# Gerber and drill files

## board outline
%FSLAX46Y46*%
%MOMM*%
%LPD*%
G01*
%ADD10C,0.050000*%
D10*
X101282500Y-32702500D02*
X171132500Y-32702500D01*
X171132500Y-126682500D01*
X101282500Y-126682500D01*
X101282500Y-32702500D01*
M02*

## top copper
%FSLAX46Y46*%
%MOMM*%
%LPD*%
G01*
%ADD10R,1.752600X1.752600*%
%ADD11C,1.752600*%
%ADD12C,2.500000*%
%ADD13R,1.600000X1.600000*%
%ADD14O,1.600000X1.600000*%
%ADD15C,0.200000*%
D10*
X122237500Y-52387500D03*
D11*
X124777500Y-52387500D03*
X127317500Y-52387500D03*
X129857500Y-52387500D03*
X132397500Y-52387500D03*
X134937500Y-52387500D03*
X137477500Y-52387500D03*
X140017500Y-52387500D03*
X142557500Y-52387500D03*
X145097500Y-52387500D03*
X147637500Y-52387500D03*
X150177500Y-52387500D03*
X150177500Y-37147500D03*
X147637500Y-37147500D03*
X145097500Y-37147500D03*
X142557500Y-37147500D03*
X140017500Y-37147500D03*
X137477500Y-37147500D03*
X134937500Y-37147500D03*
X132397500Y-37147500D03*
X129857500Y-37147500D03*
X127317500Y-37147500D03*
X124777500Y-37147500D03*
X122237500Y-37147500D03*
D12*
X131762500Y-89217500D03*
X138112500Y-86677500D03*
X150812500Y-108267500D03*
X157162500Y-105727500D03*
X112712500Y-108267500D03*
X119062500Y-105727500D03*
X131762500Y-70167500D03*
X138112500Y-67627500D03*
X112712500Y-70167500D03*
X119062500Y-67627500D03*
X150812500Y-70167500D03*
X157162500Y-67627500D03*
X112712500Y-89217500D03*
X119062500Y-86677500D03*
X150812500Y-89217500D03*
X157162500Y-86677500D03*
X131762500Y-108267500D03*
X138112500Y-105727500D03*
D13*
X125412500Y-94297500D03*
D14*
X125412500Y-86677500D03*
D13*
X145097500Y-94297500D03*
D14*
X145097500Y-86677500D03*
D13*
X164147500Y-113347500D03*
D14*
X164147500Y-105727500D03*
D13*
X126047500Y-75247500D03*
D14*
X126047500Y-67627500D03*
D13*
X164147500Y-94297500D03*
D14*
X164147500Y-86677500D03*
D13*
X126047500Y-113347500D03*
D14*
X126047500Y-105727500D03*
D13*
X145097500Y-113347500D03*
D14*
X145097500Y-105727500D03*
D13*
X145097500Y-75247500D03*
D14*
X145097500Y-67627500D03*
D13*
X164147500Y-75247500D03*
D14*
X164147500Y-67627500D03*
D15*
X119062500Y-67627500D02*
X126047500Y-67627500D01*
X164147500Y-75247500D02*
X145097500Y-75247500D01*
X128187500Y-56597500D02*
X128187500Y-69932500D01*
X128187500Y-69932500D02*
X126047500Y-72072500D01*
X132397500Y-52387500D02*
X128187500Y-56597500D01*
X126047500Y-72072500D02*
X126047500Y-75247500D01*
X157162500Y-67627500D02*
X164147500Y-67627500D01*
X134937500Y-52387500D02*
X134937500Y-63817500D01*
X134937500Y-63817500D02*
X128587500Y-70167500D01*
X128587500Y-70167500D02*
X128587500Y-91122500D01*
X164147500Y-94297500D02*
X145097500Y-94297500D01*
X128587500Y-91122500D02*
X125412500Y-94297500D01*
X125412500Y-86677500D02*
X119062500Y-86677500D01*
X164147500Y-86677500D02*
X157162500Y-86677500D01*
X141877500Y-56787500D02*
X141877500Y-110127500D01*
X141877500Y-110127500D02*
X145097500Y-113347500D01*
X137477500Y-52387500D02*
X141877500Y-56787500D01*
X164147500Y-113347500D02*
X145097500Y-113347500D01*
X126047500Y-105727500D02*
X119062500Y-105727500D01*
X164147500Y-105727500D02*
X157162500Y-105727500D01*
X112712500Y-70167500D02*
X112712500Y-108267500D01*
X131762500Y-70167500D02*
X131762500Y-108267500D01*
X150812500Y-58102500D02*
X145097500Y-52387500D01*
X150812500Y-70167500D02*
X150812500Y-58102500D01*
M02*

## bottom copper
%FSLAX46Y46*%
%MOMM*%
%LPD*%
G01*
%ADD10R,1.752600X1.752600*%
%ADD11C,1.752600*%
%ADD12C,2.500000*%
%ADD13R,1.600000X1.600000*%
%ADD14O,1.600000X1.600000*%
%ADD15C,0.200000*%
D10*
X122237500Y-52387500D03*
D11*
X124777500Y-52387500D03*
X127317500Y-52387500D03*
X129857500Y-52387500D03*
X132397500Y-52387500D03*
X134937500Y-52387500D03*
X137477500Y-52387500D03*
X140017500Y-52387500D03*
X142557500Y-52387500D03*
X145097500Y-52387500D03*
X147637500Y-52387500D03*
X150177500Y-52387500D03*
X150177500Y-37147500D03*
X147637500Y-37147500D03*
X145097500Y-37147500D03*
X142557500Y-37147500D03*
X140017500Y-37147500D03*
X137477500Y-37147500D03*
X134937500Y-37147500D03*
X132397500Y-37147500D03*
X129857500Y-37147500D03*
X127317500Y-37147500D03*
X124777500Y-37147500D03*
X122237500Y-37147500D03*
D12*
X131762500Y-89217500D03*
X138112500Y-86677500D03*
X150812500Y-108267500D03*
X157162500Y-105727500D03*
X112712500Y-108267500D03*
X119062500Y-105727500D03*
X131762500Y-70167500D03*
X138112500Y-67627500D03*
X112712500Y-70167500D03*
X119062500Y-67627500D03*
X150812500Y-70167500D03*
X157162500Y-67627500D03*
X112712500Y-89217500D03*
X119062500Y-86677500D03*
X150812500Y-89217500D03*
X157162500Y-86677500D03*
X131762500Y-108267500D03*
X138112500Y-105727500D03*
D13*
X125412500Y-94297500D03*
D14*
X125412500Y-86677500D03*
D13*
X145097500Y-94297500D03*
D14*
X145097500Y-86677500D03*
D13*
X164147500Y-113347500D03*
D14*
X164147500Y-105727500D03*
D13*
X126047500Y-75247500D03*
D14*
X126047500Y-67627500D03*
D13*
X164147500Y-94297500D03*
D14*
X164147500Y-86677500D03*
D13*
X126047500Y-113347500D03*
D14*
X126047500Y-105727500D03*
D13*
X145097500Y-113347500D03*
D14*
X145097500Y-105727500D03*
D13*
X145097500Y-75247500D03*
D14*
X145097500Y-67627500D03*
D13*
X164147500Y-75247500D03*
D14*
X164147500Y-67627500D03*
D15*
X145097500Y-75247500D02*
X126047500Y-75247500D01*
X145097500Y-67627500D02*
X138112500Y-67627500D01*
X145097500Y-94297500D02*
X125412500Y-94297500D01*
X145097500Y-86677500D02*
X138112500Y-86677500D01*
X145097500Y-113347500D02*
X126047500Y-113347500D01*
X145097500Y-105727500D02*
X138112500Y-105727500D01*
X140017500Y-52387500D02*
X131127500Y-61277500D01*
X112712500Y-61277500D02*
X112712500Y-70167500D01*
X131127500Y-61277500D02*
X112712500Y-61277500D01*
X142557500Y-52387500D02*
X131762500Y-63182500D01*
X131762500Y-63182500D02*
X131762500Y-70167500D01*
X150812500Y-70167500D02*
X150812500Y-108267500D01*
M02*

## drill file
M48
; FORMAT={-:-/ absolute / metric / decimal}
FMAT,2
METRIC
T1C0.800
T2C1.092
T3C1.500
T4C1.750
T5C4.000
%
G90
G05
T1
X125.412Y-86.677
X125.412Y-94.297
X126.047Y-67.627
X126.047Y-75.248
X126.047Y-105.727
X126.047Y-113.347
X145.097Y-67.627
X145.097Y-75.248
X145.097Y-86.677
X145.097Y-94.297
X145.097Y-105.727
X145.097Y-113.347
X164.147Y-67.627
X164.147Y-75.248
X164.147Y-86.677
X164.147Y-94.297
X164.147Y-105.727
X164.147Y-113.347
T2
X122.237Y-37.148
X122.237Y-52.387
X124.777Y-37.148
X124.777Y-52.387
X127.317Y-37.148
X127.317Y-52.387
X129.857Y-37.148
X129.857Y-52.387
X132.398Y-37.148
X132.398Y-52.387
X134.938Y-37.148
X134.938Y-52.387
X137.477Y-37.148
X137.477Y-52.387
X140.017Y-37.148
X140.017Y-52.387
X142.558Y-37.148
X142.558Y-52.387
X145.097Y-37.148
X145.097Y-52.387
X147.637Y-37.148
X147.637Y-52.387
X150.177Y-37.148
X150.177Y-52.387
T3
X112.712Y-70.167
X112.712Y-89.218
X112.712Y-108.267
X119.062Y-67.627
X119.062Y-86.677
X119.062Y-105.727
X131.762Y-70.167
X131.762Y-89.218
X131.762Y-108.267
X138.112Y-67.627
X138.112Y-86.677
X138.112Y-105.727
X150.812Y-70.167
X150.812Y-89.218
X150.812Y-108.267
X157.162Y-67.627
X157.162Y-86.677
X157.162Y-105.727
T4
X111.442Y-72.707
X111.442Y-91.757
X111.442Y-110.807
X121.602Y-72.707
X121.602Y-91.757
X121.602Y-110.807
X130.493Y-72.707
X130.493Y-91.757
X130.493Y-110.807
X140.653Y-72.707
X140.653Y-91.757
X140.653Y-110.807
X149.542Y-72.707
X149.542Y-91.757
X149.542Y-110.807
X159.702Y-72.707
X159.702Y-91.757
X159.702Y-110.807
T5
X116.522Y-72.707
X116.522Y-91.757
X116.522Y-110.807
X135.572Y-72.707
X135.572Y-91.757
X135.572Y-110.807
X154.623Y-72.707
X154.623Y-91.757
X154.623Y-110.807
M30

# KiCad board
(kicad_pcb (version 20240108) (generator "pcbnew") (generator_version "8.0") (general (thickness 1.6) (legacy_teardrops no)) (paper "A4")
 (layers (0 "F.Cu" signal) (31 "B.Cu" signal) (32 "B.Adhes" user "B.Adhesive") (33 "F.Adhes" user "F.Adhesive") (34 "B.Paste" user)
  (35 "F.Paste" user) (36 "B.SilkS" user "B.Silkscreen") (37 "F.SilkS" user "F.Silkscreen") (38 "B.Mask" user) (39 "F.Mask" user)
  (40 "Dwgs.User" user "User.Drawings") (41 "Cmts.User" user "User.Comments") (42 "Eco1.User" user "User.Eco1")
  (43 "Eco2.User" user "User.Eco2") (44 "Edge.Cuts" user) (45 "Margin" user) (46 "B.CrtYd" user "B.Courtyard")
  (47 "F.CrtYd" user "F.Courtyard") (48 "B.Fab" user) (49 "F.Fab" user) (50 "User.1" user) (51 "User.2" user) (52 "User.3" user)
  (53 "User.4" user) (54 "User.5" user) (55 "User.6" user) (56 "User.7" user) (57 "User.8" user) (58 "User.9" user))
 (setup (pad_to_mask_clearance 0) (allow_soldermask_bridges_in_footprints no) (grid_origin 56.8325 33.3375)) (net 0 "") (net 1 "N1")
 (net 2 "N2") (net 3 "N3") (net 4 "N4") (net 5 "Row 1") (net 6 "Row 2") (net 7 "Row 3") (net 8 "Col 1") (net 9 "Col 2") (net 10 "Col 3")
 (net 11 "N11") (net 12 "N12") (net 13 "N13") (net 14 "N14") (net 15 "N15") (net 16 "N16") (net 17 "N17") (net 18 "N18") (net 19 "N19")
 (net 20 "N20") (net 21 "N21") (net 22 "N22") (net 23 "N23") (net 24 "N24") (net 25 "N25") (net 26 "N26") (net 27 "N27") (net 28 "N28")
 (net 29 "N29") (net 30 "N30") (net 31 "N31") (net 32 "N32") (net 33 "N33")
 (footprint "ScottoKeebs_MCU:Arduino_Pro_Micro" (layer "F.Cu") (at 136.2075 44.7675 90)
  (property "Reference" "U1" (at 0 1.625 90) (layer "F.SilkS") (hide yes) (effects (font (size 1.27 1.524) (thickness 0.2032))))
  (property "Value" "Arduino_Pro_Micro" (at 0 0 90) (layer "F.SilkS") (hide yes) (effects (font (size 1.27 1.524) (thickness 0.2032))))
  (pad "1" thru_hole rect (at -7.62 -13.97) (size 1.7526 1.7526) (drill 1.0922) (layers "*.Cu" "*.SilkS" "*.Mask") (remove_unused_layers no)
   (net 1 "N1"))
  (pad "2" thru_hole circle (at -7.62 -11.43) (size 1.7526 1.7526) (drill 1.0922) (layers "*.Cu" "*.SilkS" "*.Mask")
   (remove_unused_layers no) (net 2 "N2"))
  (pad "3" thru_hole circle (at -7.62 -8.89) (size 1.7526 1.7526) (drill 1.0922) (layers "*.Cu" "*.SilkS" "*.Mask")
   (remove_unused_layers no) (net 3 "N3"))
  (pad "4" thru_hole circle (at -7.62 -6.35) (size 1.7526 1.7526) (drill 1.0922) (layers "*.Cu" "*.SilkS" "*.Mask")
   (remove_unused_layers no) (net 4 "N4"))
  (pad "5" thru_hole circle (at -7.62 -3.81) (size 1.7526 1.7526) (drill 1.0922) (layers "*.Cu" "*.SilkS" "*.Mask")
   (remove_unused_layers no) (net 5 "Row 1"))
  (pad "6" thru_hole circle (at -7.62 -1.27) (size 1.7526 1.7526) (drill 1.0922) (layers "*.Cu" "*.SilkS" "*.Mask")
   (remove_unused_layers no) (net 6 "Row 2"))
  (pad "7" thru_hole circle (at -7.62 1.27) (size 1.7526 1.7526) (drill 1.0922) (layers "*.Cu" "*.SilkS" "*.Mask") (remove_unused_layers no)
   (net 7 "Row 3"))
  (pad "8" thru_hole circle (at -7.62 3.81) (size 1.7526 1.7526) (drill 1.0922) (layers "*.Cu" "*.SilkS" "*.Mask") (remove_unused_layers no)
   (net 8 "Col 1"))
  (pad "9" thru_hole circle (at -7.62 6.35) (size 1.7526 1.7526) (drill 1.0922) (layers "*.Cu" "*.SilkS" "*.Mask") (remove_unused_layers no)
   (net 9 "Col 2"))
  (pad "10" thru_hole circle (at -7.62 8.89) (size 1.7526 1.7526) (drill 1.0922) (layers "*.Cu" "*.SilkS" "*.Mask")
   (remove_unused_layers no) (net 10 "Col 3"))
  (pad "11" thru_hole circle (at -7.62 11.43) (size 1.7526 1.7526) (drill 1.0922) (layers "*.Cu" "*.SilkS" "*.Mask")
   (remove_unused_layers no) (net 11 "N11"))
  (pad "12" thru_hole circle (at -7.62 13.97) (size 1.7526 1.7526) (drill 1.0922) (layers "*.Cu" "*.SilkS" "*.Mask")
   (remove_unused_layers no) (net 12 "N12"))
  (pad "13" thru_hole circle (at 7.62 13.97) (size 1.7526 1.7526) (drill 1.0922) (layers "*.Cu" "*.SilkS" "*.Mask")
   (remove_unused_layers no) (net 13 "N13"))
  (pad "14" thru_hole circle (at 7.62 11.43) (size 1.7526 1.7526) (drill 1.0922) (layers "*.Cu" "*.SilkS" "*.Mask")
   (remove_unused_layers no) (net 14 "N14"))
  (pad "15" thru_hole circle (at 7.62 8.89) (size 1.7526 1.7526) (drill 1.0922) (layers "*.Cu" "*.SilkS" "*.Mask") (remove_unused_layers no)
   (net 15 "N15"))
  (pad "16" thru_hole circle (at 7.62 6.35) (size 1.7526 1.7526) (drill 1.0922) (layers "*.Cu" "*.SilkS" "*.Mask") (remove_unused_layers no)
   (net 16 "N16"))
  (pad "17" thru_hole circle (at 7.62 3.81) (size 1.7526 1.7526) (drill 1.0922) (layers "*.Cu" "*.SilkS" "*.Mask") (remove_unused_layers no)
   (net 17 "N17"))
  (pad "18" thru_hole circle (at 7.62 1.27) (size 1.7526 1.7526) (drill 1.0922) (layers "*.Cu" "*.SilkS" "*.Mask") (remove_unused_layers no)
   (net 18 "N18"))
  (pad "19" thru_hole circle (at 7.62 -1.27) (size 1.7526 1.7526) (drill 1.0922) (layers "*.Cu" "*.SilkS" "*.Mask")
   (remove_unused_layers no) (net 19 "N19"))
  (pad "20" thru_hole circle (at 7.62 -3.81) (size 1.7526 1.7526) (drill 1.0922) (layers "*.Cu" "*.SilkS" "*.Mask")
   (remove_unused_layers no) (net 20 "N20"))
  (pad "21" thru_hole circle (at 7.62 -6.35) (size 1.7526 1.7526) (drill 1.0922) (layers "*.Cu" "*.SilkS" "*.Mask")
   (remove_unused_layers no) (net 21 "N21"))
  (pad "22" thru_hole circle (at 7.62 -8.89) (size 1.7526 1.7526) (drill 1.0922) (layers "*.Cu" "*.SilkS" "*.Mask")
   (remove_unused_layers no) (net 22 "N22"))
  (pad "23" thru_hole circle (at 7.62 -11.43) (size 1.7526 1.7526) (drill 1.0922) (layers "*.Cu" "*.SilkS" "*.Mask")
   (remove_unused_layers no) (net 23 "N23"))
  (pad "24" thru_hole circle (at 7.62 -13.97) (size 1.7526 1.7526) (drill 1.0922) (layers "*.Cu" "*.SilkS" "*.Mask")
   (remove_unused_layers no) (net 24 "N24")))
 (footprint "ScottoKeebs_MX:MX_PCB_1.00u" (layer "F.Cu") (at 135.5725 91.7575)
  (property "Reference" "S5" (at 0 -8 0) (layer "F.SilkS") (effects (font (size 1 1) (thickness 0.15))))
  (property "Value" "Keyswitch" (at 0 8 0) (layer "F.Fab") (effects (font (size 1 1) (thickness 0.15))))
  (pad "" np_thru_hole circle (at -5.08 0) (size 1.75 1.75) (drill 1.75) (layers "*.Cu" "*.Mask"))
  (pad "" np_thru_hole circle (at 0 0) (size 4 4) (drill 4) (layers "*.Cu" "*.Mask"))
  (pad "" np_thru_hole circle (at 5.08 0) (size 1.75 1.75) (drill 1.75) (layers "*.Cu" "*.Mask"))
  (pad "1" thru_hole circle (at -3.81 -2.54) (size 2.5 2.5) (drill 1.5) (layers "*.Cu" "*.Mask") (remove_unused_layers no) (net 9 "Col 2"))
  (pad "2" thru_hole circle (at 2.54 -5.08) (size 2.5 2.5) (drill 1.5) (layers "*.Cu" "*.Mask") (remove_unused_layers no) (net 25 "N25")))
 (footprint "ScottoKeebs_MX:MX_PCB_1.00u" (layer "F.Cu") (at 154.6225 110.8075)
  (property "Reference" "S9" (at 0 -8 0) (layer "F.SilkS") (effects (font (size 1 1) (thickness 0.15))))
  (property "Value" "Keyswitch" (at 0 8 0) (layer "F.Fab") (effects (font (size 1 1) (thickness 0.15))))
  (pad "" np_thru_hole circle (at -5.08 0) (size 1.75 1.75) (drill 1.75) (layers "*.Cu" "*.Mask"))
  (pad "" np_thru_hole circle (at 0 0) (size 4 4) (drill 4) (layers "*.Cu" "*.Mask"))
  (pad "" np_thru_hole circle (at 5.08 0) (size 1.75 1.75) (drill 1.75) (layers "*.Cu" "*.Mask"))
  (pad "1" thru_hole circle (at -3.81 -2.54) (size 2.5 2.5) (drill 1.5) (layers "*.Cu" "*.Mask") (remove_unused_layers no) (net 10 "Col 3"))
  (pad "2" thru_hole circle (at 2.54 -5.08) (size 2.5 2.5) (drill 1.5) (layers "*.Cu" "*.Mask") (remove_unused_layers no) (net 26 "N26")))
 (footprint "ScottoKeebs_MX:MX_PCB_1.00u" (layer "F.Cu") (at 116.5225 110.8075)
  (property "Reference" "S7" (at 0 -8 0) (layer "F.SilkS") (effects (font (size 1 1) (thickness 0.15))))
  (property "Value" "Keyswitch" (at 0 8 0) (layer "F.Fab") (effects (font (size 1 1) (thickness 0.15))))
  (pad "" np_thru_hole circle (at -5.08 0) (size 1.75 1.75) (drill 1.75) (layers "*.Cu" "*.Mask"))
  (pad "" np_thru_hole circle (at 0 0) (size 4 4) (drill 4) (layers "*.Cu" "*.Mask"))
  (pad "" np_thru_hole circle (at 5.08 0) (size 1.75 1.75) (drill 1.75) (layers "*.Cu" "*.Mask"))
  (pad "1" thru_hole circle (at -3.81 -2.54) (size 2.5 2.5) (drill 1.5) (layers "*.Cu" "*.Mask") (remove_unused_layers no) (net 8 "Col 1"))
  (pad "2" thru_hole circle (at 2.54 -5.08) (size 2.5 2.5) (drill 1.5) (layers "*.Cu" "*.Mask") (remove_unused_layers no) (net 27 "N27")))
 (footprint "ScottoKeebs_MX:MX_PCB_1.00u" (layer "F.Cu") (at 135.5725 72.7075)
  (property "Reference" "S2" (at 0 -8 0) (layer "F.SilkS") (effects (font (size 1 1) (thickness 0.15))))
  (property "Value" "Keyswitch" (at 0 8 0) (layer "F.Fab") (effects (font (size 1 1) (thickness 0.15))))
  (pad "" np_thru_hole circle (at -5.08 0) (size 1.75 1.75) (drill 1.75) (layers "*.Cu" "*.Mask"))
  (pad "" np_thru_hole circle (at 0 0) (size 4 4) (drill 4) (layers "*.Cu" "*.Mask"))
  (pad "" np_thru_hole circle (at 5.08 0) (size 1.75 1.75) (drill 1.75) (layers "*.Cu" "*.Mask"))
  (pad "1" thru_hole circle (at -3.81 -2.54) (size 2.5 2.5) (drill 1.5) (layers "*.Cu" "*.Mask") (remove_unused_layers no) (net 9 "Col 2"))
  (pad "2" thru_hole circle (at 2.54 -5.08) (size 2.5 2.5) (drill 1.5) (layers "*.Cu" "*.Mask") (remove_unused_layers no) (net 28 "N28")))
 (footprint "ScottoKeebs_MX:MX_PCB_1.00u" (layer "F.Cu") (at 116.5225 72.7075)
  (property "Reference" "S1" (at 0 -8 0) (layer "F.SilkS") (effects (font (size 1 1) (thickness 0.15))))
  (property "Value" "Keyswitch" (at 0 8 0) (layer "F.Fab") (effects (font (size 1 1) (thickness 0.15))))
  (pad "" np_thru_hole circle (at -5.08 0) (size 1.75 1.75) (drill 1.75) (layers "*.Cu" "*.Mask"))
  (pad "" np_thru_hole circle (at 0 0) (size 4 4) (drill 4) (layers "*.Cu" "*.Mask"))
  (pad "" np_thru_hole circle (at 5.08 0) (size 1.75 1.75) (drill 1.75) (layers "*.Cu" "*.Mask"))
  (pad "1" thru_hole circle (at -3.81 -2.54) (size 2.5 2.5) (drill 1.5) (layers "*.Cu" "*.Mask") (remove_unused_layers no) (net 8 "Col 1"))
  (pad "2" thru_hole circle (at 2.54 -5.08) (size 2.5 2.5) (drill 1.5) (layers "*.Cu" "*.Mask") (remove_unused_layers no) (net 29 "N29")))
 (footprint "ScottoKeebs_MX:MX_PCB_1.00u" (layer "F.Cu") (at 154.6225 72.7075)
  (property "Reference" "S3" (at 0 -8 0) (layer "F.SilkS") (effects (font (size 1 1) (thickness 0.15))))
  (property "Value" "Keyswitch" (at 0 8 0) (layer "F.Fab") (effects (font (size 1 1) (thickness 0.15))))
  (pad "" np_thru_hole circle (at -5.08 0) (size 1.75 1.75) (drill 1.75) (layers "*.Cu" "*.Mask"))
  (pad "" np_thru_hole circle (at 0 0) (size 4 4) (drill 4) (layers "*.Cu" "*.Mask"))
  (pad "" np_thru_hole circle (at 5.08 0) (size 1.75 1.75) (drill 1.75) (layers "*.Cu" "*.Mask"))
  (pad "1" thru_hole circle (at -3.81 -2.54) (size 2.5 2.5) (drill 1.5) (layers "*.Cu" "*.Mask") (remove_unused_layers no) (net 10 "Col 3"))
  (pad "2" thru_hole circle (at 2.54 -5.08) (size 2.5 2.5) (drill 1.5) (layers "*.Cu" "*.Mask") (remove_unused_layers no) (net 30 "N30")))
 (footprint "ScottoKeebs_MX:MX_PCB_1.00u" (layer "F.Cu") (at 116.5225 91.7575)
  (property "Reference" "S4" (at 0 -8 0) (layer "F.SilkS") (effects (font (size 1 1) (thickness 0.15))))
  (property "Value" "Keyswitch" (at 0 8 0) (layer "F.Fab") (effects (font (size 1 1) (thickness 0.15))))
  (pad "" np_thru_hole circle (at -5.08 0) (size 1.75 1.75) (drill 1.75) (layers "*.Cu" "*.Mask"))
  (pad "" np_thru_hole circle (at 0 0) (size 4 4) (drill 4) (layers "*.Cu" "*.Mask"))
  (pad "" np_thru_hole circle (at 5.08 0) (size 1.75 1.75) (drill 1.75) (layers "*.Cu" "*.Mask"))
  (pad "1" thru_hole circle (at -3.81 -2.54) (size 2.5 2.5) (drill 1.5) (layers "*.Cu" "*.Mask") (remove_unused_layers no) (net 8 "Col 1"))
  (pad "2" thru_hole circle (at 2.54 -5.08) (size 2.5 2.5) (drill 1.5) (layers "*.Cu" "*.Mask") (remove_unused_layers no) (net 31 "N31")))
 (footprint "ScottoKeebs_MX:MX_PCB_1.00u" (layer "F.Cu") (at 154.6225 91.7575)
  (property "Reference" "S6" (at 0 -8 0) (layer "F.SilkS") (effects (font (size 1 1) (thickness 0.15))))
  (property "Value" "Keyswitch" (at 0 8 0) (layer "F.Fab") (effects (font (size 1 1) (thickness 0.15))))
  (pad "" np_thru_hole circle (at -5.08 0) (size 1.75 1.75) (drill 1.75) (layers "*.Cu" "*.Mask"))
  (pad "" np_thru_hole circle (at 0 0) (size 4 4) (drill 4) (layers "*.Cu" "*.Mask"))
  (pad "" np_thru_hole circle (at 5.08 0) (size 1.75 1.75) (drill 1.75) (layers "*.Cu" "*.Mask"))
  (pad "1" thru_hole circle (at -3.81 -2.54) (size 2.5 2.5) (drill 1.5) (layers "*.Cu" "*.Mask") (remove_unused_layers no) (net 10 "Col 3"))
  (pad "2" thru_hole circle (at 2.54 -5.08) (size 2.5 2.5) (drill 1.5) (layers "*.Cu" "*.Mask") (remove_unused_layers no) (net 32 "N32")))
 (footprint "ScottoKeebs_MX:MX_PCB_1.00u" (layer "F.Cu") (at 135.5725 110.8075)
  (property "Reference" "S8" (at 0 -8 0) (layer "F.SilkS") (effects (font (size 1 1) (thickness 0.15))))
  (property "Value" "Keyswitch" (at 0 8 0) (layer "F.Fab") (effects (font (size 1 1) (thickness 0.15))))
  (pad "" np_thru_hole circle (at -5.08 0) (size 1.75 1.75) (drill 1.75) (layers "*.Cu" "*.Mask"))
  (pad "" np_thru_hole circle (at 0 0) (size 4 4) (drill 4) (layers "*.Cu" "*.Mask"))
  (pad "" np_thru_hole circle (at 5.08 0) (size 1.75 1.75) (drill 1.75) (layers "*.Cu" "*.Mask"))
  (pad "1" thru_hole circle (at -3.81 -2.54) (size 2.5 2.5) (drill 1.5) (layers "*.Cu" "*.Mask") (remove_unused_layers no) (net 9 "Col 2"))
  (pad "2" thru_hole circle (at 2.54 -5.08) (size 2.5 2.5) (drill 1.5) (layers "*.Cu" "*.Mask") (remove_unused_layers no) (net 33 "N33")))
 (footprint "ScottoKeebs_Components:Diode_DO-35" (layer "B.Cu") (at 125.4125 94.2975 90)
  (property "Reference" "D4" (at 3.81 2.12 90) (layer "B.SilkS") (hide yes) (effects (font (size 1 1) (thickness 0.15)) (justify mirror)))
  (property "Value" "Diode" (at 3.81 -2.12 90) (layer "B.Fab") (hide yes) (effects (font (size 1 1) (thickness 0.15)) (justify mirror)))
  (pad "1" thru_hole rect (at 0 0 90) (size 1.6 1.6) (drill 0.8) (layers "*.Cu" "*.Mask") (remove_unused_layers no) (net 6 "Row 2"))
  (pad "2" thru_hole oval (at 7.62 0 90) (size 1.6 1.6) (drill 0.8) (layers "*.Cu" "*.Mask") (remove_unused_layers no) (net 31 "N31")))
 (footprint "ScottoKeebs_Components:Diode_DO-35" (layer "B.Cu") (at 145.0975 94.2975 90)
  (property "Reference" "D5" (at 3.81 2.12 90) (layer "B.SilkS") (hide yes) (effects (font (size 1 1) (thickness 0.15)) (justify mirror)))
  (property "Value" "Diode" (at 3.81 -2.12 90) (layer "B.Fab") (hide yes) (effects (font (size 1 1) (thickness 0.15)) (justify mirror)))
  (pad "1" thru_hole rect (at 0 0 90) (size 1.6 1.6) (drill 0.8) (layers "*.Cu" "*.Mask") (remove_unused_layers no) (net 6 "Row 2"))
  (pad "2" thru_hole oval (at 7.62 0 90) (size 1.6 1.6) (drill 0.8) (layers "*.Cu" "*.Mask") (remove_unused_layers no) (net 25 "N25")))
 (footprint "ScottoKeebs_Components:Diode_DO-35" (layer "B.Cu") (at 164.1475 113.3475 90)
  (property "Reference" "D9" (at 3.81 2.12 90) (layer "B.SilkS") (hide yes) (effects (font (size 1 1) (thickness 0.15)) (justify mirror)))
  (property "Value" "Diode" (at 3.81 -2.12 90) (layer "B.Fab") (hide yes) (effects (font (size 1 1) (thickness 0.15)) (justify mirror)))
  (pad "1" thru_hole rect (at 0 0 90) (size 1.6 1.6) (drill 0.8) (layers "*.Cu" "*.Mask") (remove_unused_layers no) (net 7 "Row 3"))
  (pad "2" thru_hole oval (at 7.62 0 90) (size 1.6 1.6) (drill 0.8) (layers "*.Cu" "*.Mask") (remove_unused_layers no) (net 26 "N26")))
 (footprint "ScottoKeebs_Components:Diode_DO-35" (layer "B.Cu") (at 126.0475 75.2475 90)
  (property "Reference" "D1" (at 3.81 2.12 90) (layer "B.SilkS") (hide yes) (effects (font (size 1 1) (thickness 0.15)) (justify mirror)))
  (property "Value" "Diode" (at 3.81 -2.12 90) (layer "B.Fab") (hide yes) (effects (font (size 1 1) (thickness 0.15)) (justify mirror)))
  (pad "1" thru_hole rect (at 0 0 90) (size 1.6 1.6) (drill 0.8) (layers "*.Cu" "*.Mask") (remove_unused_layers no) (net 5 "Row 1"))
  (pad "2" thru_hole oval (at 7.62 0 90) (size 1.6 1.6) (drill 0.8) (layers "*.Cu" "*.Mask") (remove_unused_layers no) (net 29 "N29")))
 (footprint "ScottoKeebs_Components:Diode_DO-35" (layer "B.Cu") (at 164.1475 94.2975 90)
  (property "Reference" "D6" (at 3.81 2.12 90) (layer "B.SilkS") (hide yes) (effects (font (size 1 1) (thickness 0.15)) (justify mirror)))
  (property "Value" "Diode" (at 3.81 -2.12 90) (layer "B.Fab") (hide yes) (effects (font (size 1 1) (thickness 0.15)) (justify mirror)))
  (pad "1" thru_hole rect (at 0 0 90) (size 1.6 1.6) (drill 0.8) (layers "*.Cu" "*.Mask") (remove_unused_layers no) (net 6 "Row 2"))
  (pad "2" thru_hole oval (at 7.62 0 90) (size 1.6 1.6) (drill 0.8) (layers "*.Cu" "*.Mask") (remove_unused_layers no) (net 32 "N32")))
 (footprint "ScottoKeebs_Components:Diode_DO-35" (layer "B.Cu") (at 126.0475 113.3475 90)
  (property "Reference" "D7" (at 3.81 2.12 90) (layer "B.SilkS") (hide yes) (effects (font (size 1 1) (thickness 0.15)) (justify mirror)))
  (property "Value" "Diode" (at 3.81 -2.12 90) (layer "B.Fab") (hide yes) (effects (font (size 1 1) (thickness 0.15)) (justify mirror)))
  (pad "1" thru_hole rect (at 0 0 90) (size 1.6 1.6) (drill 0.8) (layers "*.Cu" "*.Mask") (remove_unused_layers no) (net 7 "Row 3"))
  (pad "2" thru_hole oval (at 7.62 0 90) (size 1.6 1.6) (drill 0.8) (layers "*.Cu" "*.Mask") (remove_unused_layers no) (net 27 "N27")))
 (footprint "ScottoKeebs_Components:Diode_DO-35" (layer "B.Cu") (at 145.0975 113.3475 90)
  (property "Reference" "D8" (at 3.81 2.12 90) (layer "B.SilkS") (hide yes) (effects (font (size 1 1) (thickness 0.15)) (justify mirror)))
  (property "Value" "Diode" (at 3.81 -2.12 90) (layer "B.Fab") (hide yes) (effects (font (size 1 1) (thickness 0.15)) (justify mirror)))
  (pad "1" thru_hole rect (at 0 0 90) (size 1.6 1.6) (drill 0.8) (layers "*.Cu" "*.Mask") (remove_unused_layers no) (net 7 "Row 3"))
  (pad "2" thru_hole oval (at 7.62 0 90) (size 1.6 1.6) (drill 0.8) (layers "*.Cu" "*.Mask") (remove_unused_layers no) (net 33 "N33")))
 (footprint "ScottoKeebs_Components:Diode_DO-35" (layer "B.Cu") (at 145.0975 75.2475 90)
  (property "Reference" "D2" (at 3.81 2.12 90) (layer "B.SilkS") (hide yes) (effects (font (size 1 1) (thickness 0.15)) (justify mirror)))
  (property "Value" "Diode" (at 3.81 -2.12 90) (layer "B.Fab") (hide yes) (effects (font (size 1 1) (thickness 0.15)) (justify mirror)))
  (pad "1" thru_hole rect (at 0 0 90) (size 1.6 1.6) (drill 0.8) (layers "*.Cu" "*.Mask") (remove_unused_layers no) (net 5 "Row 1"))
  (pad "2" thru_hole oval (at 7.62 0 90) (size 1.6 1.6) (drill 0.8) (layers "*.Cu" "*.Mask") (remove_unused_layers no) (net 28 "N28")))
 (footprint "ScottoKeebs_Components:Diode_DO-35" (layer "B.Cu") (at 164.1475 75.2475 90)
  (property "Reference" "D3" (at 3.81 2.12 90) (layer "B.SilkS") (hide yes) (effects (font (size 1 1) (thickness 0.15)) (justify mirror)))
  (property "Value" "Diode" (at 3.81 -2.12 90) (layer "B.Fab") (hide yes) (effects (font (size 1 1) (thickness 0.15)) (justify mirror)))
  (pad "1" thru_hole rect (at 0 0 90) (size 1.6 1.6) (drill 0.8) (layers "*.Cu" "*.Mask") (remove_unused_layers no) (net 5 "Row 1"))
  (pad "2" thru_hole oval (at 7.62 0 90) (size 1.6 1.6) (drill 0.8) (layers "*.Cu" "*.Mask") (remove_unused_layers no) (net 30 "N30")))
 (gr_rect (start 101.2825 32.7025) (end 171.1325 126.6825) (stroke (width 0.05) (type default)) (fill none) (layer "Edge.Cuts"))
 (segment (start 119.0625 67.6275) (end 126.0475 67.6275) (width 0.2) (layer "F.Cu") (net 29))
 (segment (start 164.1475 75.2475) (end 145.0975 75.2475) (width 0.2) (layer "F.Cu") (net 5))
 (segment (start 128.1875 56.5975) (end 128.1875 69.9325) (width 0.2) (layer "F.Cu") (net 5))
 (segment (start 128.1875 69.9325) (end 126.0475 72.0725) (width 0.2) (layer "F.Cu") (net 5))
 (segment (start 132.3975 52.3875) (end 128.1875 56.5975) (width 0.2) (layer "F.Cu") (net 5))
 (segment (start 126.0475 72.0725) (end 126.0475 75.2475) (width 0.2) (layer "F.Cu") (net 5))
 (segment (start 145.0975 75.2475) (end 126.0475 75.2475) (width 0.2) (layer "B.Cu") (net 5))
 (segment (start 145.0975 67.6275) (end 138.1125 67.6275) (width 0.2) (layer "B.Cu") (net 28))
 (segment (start 157.1625 67.6275) (end 164.1475 67.6275) (width 0.2) (layer "F.Cu") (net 30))
 (segment (start 134.9375 52.3875) (end 134.9375 63.8175) (width 0.2) (layer "F.Cu") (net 6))
 (segment (start 134.9375 63.8175) (end 128.5875 70.1675) (width 0.2) (layer "F.Cu") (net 6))
 (segment (start 128.5875 70.1675) (end 128.5875 91.1225) (width 0.2) (layer "F.Cu") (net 6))
 (segment (start 164.1475 94.2975) (end 145.0975 94.2975) (width 0.2) (layer "F.Cu") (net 6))
 (segment (start 128.5875 91.1225) (end 125.4125 94.2975) (width 0.2) (layer "F.Cu") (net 6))
 (segment (start 145.0975 94.2975) (end 125.4125 94.2975) (width 0.2) (layer "B.Cu") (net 6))
 (segment (start 125.4125 86.6775) (end 119.0625 86.6775) (width 0.2) (layer "F.Cu") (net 31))
 (segment (start 145.0975 86.6775) (end 138.1125 86.6775) (width 0.2) (layer "B.Cu") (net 25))
 (segment (start 164.1475 86.6775) (end 157.1625 86.6775) (width 0.2) (layer "F.Cu") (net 32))
 (segment (start 141.8775 56.7875) (end 141.8775 110.1275) (width 0.2) (layer "F.Cu") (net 7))
 (segment (start 141.8775 110.1275) (end 145.0975 113.3475) (width 0.2) (layer "F.Cu") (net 7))
 (segment (start 137.4775 52.3875) (end 141.8775 56.7875) (width 0.2) (layer "F.Cu") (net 7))
 (segment (start 164.1475 113.3475) (end 145.0975 113.3475) (width 0.2) (layer "F.Cu") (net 7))
 (segment (start 145.0975 113.3475) (end 126.0475 113.3475) (width 0.2) (layer "B.Cu") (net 7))
 (segment (start 126.0475 105.7275) (end 119.0625 105.7275) (width 0.2) (layer "F.Cu") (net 27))
 (segment (start 145.0975 105.7275) (end 138.1125 105.7275) (width 0.2) (layer "B.Cu") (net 33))
 (segment (start 164.1475 105.7275) (end 157.1625 105.7275) (width 0.2) (layer "F.Cu") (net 26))
 (segment (start 112.7125 70.1675) (end 112.7125 108.2675) (width 0.2) (layer "F.Cu") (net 8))
 (segment (start 140.0175 52.3875) (end 131.1275 61.2775) (width 0.2) (layer "B.Cu") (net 8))
 (segment (start 112.7125 61.2775) (end 112.7125 70.1675) (width 0.2) (layer "B.Cu") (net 8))
 (segment (start 131.1275 61.2775) (end 112.7125 61.2775) (width 0.2) (layer "B.Cu") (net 8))
 (segment (start 131.7625 70.1675) (end 131.7625 108.2675) (width 0.2) (layer "F.Cu") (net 9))
 (segment (start 142.5575 52.3875) (end 131.7625 63.1825) (width 0.2) (layer "B.Cu") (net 9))
 (segment (start 131.7625 63.1825) (end 131.7625 70.1675) (width 0.2) (layer "B.Cu") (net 9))
 (segment (start 150.8125 58.1025) (end 145.0975 52.3875) (width 0.2) (layer "F.Cu") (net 10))
 (segment (start 150.8125 70.1675) (end 150.8125 58.1025) (width 0.2) (layer "F.Cu") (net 10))
 (segment (start 150.8125 70.1675) (end 150.8125 108.2675) (width 0.2) (layer "B.Cu") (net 10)))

